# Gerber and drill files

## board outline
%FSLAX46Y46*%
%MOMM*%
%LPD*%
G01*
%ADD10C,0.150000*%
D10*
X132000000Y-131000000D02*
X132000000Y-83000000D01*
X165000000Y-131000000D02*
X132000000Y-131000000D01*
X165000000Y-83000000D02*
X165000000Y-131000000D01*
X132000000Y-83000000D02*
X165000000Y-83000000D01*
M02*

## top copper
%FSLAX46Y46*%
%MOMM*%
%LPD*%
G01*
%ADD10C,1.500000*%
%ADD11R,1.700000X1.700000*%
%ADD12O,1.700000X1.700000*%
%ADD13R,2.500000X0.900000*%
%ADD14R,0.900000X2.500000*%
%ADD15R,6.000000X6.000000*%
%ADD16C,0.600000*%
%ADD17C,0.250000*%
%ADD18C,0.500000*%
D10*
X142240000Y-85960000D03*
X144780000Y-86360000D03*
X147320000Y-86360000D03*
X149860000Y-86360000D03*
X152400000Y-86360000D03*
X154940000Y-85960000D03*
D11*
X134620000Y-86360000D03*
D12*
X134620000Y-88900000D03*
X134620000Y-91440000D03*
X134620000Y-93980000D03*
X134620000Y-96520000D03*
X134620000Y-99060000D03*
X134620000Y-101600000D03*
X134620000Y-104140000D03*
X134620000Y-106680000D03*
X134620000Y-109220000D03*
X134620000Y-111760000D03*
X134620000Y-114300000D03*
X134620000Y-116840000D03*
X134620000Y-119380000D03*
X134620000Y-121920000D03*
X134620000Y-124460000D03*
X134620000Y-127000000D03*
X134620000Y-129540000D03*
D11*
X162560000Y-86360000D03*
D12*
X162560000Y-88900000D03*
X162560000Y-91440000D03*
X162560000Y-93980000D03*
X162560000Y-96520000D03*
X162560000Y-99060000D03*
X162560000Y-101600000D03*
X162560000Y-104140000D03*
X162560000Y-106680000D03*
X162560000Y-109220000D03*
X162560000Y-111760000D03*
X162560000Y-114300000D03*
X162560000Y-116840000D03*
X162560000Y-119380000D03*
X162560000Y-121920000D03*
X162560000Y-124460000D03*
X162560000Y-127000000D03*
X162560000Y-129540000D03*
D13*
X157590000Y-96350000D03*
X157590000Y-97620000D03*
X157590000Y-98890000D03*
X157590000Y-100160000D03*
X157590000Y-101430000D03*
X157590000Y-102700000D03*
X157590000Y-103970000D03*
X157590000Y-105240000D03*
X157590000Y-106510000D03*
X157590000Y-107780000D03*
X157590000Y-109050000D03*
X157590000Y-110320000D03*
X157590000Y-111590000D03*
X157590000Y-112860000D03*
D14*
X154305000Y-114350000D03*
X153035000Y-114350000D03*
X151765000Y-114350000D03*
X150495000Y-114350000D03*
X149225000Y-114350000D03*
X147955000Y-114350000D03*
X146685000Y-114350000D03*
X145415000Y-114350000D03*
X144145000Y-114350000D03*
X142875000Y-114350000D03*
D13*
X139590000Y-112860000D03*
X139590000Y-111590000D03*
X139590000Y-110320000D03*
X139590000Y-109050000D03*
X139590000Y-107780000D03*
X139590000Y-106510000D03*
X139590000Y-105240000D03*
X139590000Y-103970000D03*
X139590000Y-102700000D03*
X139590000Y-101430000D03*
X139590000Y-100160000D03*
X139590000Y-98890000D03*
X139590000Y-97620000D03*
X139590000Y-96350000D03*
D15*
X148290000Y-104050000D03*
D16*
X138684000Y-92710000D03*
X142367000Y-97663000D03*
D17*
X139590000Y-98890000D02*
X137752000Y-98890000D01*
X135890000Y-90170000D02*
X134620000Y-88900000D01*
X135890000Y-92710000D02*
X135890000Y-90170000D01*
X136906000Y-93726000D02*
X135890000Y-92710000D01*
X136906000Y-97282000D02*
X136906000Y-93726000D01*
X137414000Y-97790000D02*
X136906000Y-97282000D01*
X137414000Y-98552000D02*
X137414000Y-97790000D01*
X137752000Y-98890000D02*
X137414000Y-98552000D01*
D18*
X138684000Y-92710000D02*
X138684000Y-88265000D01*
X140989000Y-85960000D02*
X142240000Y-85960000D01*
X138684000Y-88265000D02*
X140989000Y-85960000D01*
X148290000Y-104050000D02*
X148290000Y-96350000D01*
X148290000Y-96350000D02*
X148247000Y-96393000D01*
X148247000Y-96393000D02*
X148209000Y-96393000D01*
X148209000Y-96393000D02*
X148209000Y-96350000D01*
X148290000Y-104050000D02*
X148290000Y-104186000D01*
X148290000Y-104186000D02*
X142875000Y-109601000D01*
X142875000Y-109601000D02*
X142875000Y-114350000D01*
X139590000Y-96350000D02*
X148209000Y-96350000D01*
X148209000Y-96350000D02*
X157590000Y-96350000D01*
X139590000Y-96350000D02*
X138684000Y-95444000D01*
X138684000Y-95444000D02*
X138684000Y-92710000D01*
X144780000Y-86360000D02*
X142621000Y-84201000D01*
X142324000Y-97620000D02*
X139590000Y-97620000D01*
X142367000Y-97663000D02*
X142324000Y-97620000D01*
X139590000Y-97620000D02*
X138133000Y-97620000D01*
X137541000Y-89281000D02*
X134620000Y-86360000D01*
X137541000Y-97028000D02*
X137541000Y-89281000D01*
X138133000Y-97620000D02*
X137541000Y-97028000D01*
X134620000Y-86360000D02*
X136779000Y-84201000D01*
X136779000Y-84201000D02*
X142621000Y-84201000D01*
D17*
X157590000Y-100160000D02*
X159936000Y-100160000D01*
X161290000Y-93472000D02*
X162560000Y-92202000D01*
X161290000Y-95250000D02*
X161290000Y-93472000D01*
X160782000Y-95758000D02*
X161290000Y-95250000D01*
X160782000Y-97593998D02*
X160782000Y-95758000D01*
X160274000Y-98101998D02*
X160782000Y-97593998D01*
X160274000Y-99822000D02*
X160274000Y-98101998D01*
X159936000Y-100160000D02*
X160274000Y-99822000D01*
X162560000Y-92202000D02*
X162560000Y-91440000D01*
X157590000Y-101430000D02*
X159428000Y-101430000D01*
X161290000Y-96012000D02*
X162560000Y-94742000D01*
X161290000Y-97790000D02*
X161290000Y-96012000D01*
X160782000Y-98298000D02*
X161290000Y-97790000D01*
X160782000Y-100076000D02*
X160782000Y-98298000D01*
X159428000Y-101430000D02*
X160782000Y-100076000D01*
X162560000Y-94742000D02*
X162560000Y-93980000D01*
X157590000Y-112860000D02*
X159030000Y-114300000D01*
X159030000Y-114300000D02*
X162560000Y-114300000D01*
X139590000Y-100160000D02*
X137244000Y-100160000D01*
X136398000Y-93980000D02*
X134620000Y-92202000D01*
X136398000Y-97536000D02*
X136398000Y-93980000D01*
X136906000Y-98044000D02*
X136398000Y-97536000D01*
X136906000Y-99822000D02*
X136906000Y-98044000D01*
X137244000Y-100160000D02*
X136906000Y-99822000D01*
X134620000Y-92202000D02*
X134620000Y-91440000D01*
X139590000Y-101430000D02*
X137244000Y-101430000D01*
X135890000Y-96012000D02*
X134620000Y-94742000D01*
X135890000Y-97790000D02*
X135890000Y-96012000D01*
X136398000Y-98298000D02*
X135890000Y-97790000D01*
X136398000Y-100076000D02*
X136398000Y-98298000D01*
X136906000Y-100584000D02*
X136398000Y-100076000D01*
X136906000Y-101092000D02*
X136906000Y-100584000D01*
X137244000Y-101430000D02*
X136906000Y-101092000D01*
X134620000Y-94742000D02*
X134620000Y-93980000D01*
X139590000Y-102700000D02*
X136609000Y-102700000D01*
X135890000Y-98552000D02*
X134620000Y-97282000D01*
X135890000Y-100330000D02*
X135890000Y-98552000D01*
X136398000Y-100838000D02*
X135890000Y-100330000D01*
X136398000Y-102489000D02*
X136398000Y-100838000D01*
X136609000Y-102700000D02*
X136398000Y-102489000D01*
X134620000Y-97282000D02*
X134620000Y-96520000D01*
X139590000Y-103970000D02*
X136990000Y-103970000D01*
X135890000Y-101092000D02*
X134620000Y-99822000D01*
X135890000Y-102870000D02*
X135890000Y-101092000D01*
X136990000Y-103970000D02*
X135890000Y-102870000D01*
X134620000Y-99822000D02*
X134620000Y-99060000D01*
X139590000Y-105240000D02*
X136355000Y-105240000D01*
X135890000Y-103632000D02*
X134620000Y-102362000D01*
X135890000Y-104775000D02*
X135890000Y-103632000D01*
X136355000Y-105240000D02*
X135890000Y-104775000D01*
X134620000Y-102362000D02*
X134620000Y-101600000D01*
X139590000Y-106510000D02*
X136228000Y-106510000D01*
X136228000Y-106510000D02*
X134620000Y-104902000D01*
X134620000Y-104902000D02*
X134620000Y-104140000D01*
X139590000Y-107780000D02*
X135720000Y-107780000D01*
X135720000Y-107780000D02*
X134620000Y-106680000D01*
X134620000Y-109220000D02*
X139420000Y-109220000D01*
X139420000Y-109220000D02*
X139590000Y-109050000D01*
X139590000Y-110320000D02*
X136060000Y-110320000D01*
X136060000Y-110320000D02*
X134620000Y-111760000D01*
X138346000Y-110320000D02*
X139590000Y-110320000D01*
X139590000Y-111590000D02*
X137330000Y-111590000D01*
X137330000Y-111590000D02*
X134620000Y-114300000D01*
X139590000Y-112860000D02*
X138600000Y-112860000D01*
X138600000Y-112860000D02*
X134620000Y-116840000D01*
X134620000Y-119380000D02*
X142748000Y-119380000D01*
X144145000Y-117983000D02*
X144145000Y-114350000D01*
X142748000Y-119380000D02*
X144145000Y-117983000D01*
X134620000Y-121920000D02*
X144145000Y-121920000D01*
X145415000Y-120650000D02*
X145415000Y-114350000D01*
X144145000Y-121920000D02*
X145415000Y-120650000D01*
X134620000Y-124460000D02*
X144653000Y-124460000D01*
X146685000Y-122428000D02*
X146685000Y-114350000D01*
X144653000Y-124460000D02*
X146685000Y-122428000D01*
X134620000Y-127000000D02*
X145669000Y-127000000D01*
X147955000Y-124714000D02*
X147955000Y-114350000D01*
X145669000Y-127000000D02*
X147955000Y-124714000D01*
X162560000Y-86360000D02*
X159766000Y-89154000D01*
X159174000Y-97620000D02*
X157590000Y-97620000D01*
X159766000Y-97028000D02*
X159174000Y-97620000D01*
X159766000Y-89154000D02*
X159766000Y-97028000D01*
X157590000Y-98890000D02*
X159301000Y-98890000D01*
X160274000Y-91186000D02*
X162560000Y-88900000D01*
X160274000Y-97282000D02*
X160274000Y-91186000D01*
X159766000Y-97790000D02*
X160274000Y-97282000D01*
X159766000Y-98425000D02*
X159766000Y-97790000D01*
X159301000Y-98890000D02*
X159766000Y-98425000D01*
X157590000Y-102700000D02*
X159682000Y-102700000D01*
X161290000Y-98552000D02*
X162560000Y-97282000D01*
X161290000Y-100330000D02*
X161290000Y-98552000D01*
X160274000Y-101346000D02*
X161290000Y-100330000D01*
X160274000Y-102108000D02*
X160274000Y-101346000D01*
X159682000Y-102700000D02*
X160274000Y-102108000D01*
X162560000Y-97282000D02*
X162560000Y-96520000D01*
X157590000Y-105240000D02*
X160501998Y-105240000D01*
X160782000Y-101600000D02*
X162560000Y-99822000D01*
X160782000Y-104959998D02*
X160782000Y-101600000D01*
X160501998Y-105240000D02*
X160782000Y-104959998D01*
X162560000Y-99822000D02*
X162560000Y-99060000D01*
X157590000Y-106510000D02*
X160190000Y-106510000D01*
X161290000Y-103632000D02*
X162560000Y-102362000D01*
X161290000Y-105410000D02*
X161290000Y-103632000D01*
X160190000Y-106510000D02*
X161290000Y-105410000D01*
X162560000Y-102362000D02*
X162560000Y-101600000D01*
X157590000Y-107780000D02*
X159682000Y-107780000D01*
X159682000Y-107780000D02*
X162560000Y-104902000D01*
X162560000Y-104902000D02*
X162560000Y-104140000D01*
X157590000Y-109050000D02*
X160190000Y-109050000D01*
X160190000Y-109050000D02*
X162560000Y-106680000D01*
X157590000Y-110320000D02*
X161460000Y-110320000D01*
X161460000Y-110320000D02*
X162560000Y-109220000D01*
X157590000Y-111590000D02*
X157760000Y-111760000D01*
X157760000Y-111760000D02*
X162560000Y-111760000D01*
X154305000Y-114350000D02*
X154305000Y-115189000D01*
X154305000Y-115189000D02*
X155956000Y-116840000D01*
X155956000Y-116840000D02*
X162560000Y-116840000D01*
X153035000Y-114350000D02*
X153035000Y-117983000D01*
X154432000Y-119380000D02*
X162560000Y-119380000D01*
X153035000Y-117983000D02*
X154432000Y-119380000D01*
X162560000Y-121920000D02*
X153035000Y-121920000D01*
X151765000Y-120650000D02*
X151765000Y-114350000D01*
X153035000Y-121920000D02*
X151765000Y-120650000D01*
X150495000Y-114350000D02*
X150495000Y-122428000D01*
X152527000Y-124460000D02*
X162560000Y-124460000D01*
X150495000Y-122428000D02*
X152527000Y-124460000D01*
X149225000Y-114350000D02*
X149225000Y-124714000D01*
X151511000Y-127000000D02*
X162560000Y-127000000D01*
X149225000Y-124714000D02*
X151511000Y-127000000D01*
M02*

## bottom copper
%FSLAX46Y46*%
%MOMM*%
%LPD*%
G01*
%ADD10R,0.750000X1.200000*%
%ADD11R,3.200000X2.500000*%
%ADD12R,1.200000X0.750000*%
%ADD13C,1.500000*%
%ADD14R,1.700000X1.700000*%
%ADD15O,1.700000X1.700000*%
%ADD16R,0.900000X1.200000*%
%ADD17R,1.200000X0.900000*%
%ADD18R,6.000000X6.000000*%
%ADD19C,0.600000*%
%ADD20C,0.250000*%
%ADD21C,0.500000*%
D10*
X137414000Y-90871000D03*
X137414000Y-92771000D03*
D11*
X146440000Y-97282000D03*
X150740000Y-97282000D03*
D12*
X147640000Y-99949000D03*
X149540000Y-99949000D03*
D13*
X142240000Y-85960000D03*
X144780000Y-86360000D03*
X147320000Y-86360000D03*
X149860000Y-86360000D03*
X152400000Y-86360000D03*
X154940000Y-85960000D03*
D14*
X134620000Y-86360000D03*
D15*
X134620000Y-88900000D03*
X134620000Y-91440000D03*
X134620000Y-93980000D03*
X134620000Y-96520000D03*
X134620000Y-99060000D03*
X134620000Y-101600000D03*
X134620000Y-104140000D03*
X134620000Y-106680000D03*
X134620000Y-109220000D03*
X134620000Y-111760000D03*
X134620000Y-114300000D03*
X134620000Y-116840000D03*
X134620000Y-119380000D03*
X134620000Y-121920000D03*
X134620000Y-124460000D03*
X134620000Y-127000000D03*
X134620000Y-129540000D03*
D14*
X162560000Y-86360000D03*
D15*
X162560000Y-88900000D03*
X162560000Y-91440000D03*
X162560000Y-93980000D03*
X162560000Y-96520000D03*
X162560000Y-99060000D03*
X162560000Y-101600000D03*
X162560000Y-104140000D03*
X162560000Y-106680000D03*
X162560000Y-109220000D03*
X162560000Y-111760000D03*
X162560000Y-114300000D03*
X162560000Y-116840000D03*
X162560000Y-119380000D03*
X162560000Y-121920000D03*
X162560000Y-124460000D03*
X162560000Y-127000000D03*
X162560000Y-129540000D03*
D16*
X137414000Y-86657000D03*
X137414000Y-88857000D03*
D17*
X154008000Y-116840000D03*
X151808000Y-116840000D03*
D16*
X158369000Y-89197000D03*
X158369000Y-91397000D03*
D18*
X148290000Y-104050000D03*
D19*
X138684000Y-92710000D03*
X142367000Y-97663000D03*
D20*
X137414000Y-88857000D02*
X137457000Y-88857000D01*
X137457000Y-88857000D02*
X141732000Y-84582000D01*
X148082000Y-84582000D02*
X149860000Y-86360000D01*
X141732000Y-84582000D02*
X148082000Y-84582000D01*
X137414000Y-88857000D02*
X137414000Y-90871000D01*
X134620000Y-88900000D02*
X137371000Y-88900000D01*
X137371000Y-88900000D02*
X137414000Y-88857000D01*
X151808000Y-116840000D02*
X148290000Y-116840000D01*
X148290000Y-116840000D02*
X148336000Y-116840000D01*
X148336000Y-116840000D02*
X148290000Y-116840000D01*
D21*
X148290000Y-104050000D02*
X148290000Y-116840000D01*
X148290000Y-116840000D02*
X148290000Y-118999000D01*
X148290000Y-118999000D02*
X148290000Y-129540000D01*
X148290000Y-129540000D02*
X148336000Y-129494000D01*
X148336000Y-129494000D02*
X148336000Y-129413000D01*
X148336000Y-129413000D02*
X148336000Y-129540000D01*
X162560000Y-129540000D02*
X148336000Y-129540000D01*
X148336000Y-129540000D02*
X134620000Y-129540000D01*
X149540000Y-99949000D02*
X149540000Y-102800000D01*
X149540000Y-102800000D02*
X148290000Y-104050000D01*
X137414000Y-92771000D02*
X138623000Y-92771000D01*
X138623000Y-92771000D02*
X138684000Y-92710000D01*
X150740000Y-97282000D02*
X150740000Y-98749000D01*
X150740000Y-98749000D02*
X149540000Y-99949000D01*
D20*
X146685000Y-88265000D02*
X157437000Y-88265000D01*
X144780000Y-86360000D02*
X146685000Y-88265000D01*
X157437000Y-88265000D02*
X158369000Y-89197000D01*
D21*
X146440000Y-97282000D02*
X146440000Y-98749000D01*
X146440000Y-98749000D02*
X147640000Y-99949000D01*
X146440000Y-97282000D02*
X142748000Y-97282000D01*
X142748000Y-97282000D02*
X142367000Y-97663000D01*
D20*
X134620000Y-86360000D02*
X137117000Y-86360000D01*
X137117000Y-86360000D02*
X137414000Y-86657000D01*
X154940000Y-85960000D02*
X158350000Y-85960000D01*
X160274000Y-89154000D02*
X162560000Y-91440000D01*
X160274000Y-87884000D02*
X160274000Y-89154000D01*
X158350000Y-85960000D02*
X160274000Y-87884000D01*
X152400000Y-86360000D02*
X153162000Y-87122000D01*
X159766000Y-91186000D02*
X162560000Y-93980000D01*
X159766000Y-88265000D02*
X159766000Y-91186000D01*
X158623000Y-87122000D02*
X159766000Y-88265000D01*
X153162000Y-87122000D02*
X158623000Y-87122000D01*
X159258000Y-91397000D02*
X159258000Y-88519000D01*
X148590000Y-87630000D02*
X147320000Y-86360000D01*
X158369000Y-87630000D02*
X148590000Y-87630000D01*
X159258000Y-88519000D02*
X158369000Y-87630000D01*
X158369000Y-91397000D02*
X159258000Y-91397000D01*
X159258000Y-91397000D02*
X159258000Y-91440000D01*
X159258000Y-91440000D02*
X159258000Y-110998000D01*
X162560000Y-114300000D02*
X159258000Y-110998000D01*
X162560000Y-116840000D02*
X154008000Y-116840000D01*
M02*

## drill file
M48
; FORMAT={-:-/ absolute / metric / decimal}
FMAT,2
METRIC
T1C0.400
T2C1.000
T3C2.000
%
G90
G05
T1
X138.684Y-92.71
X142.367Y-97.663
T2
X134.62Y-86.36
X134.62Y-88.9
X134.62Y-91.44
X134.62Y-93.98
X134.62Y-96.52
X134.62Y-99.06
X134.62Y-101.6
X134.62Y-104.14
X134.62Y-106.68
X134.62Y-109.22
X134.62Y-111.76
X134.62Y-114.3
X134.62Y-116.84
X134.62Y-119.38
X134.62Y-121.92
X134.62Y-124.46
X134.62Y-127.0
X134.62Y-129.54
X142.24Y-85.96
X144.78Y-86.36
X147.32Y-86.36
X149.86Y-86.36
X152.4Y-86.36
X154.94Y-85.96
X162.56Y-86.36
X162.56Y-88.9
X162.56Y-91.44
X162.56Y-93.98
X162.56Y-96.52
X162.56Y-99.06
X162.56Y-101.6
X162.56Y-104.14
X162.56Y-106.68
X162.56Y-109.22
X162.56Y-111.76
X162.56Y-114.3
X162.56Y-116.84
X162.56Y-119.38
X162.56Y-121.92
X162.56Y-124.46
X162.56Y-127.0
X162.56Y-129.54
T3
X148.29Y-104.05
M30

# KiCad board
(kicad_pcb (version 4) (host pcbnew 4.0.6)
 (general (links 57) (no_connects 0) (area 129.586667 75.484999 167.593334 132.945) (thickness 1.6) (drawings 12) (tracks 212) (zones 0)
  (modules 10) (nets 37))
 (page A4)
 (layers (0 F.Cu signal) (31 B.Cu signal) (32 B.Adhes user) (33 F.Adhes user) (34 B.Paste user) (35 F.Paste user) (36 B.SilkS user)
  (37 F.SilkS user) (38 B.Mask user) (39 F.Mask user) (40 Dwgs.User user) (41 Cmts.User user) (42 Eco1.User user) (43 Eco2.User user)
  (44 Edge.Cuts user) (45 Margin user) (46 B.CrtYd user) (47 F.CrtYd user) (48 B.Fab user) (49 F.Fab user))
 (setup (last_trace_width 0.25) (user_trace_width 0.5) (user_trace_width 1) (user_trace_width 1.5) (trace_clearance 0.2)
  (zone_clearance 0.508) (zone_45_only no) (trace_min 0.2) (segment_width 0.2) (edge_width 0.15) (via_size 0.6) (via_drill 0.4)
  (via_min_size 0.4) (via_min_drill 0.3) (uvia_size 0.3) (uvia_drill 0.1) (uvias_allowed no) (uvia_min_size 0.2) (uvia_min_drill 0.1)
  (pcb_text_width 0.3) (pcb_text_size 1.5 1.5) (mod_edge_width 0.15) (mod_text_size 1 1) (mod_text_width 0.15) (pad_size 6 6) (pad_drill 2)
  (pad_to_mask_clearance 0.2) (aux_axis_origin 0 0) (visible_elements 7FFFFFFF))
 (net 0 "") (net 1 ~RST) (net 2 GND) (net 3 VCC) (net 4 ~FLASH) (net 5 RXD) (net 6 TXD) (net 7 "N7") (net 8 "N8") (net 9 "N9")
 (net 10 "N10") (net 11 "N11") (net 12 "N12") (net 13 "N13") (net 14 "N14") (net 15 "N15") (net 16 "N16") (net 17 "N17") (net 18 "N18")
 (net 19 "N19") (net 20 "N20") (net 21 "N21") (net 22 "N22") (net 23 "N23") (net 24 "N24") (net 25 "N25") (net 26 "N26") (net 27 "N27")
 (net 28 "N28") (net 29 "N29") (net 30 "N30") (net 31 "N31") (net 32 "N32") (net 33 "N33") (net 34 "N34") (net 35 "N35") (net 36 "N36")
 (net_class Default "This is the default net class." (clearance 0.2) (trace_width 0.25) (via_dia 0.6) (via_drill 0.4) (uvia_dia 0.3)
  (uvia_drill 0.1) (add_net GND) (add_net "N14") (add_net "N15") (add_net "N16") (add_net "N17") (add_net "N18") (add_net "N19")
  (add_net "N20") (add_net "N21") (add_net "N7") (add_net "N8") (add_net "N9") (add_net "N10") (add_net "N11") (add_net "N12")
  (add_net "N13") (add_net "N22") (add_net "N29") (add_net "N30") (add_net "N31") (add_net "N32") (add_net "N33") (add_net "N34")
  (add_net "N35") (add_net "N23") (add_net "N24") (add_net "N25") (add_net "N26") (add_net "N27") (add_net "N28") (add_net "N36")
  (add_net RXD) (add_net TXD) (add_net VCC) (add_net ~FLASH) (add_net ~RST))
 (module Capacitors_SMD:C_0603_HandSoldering (layer B.Cu) (at 137.414 91.821 270)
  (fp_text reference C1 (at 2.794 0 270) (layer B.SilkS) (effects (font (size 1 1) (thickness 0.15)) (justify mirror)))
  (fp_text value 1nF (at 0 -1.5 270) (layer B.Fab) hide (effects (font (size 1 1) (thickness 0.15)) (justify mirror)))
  (pad 1 smd rect (at -0.95 0 270) (size 1.2 0.75) (layers B.Cu B.Paste B.Mask) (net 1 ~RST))
  (pad 2 smd rect (at 0.95 0 270) (size 1.2 0.75) (layers B.Cu B.Paste B.Mask) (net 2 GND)))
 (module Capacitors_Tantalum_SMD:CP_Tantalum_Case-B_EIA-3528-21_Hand (layer B.Cu) (at 148.59 97.282)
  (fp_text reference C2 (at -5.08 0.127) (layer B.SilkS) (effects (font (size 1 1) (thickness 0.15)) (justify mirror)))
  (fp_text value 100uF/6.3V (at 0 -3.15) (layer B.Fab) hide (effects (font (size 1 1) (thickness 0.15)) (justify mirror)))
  (pad 1 smd rect (at -2.15 0) (size 3.2 2.5) (layers B.Cu B.Paste B.Mask) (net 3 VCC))
  (pad 2 smd rect (at 2.15 0) (size 3.2 2.5) (layers B.Cu B.Paste B.Mask) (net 2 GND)))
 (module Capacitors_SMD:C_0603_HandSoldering (layer B.Cu) (at 148.59 99.949)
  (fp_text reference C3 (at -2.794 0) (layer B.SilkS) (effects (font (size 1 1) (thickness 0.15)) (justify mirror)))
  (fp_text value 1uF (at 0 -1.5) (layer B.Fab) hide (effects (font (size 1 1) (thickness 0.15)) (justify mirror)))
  (pad 1 smd rect (at -0.95 0) (size 1.2 0.75) (layers B.Cu B.Paste B.Mask) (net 3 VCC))
  (pad 2 smd rect (at 0.95 0) (size 1.2 0.75) (layers B.Cu B.Paste B.Mask) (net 2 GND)))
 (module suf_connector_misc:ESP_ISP (layer F.Cu) (at 142.24 86.36 90)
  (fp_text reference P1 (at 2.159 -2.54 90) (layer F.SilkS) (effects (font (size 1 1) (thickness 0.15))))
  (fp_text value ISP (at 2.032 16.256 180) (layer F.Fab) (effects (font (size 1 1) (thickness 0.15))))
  (pad 1 thru_hole circle (at 0.4 0 90) (size 1.5 1.5) (drill 1) (layers *.Cu *.Mask) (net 2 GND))
  (pad 2 thru_hole circle (at 0 2.54 90) (size 1.5 1.5) (drill 1) (layers *.Cu *.Mask) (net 3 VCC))
  (pad 3 thru_hole circle (at 0 5.08 90) (size 1.5 1.5) (drill 1) (layers *.Cu *.Mask) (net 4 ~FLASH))
  (pad 4 thru_hole circle (at 0 7.62 90) (size 1.5 1.5) (drill 1) (layers *.Cu *.Mask) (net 1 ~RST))
  (pad 5 thru_hole circle (at 0 10.16 90) (size 1.5 1.5) (drill 1) (layers *.Cu *.Mask) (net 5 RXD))
  (pad 6 thru_hole circle (at 0.4 12.7 90) (size 1.5 1.5) (drill 1) (layers *.Cu *.Mask) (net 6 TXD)))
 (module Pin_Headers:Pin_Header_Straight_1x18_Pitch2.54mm (layer F.Cu) (at 134.62 86.36)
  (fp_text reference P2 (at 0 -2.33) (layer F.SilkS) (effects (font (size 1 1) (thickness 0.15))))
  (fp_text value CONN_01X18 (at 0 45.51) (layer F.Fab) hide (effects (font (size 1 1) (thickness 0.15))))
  (pad 1 thru_hole rect (at 0 0) (size 1.7 1.7) (drill 1) (layers *.Cu *.Mask) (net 3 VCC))
  (pad 2 thru_hole oval (at 0 2.54) (size 1.7 1.7) (drill 1) (layers *.Cu *.Mask) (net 1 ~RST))
  (pad 3 thru_hole oval (at 0 5.08) (size 1.7 1.7) (drill 1) (layers *.Cu *.Mask) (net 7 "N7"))
  (pad 4 thru_hole oval (at 0 7.62) (size 1.7 1.7) (drill 1) (layers *.Cu *.Mask) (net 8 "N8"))
  (pad 5 thru_hole oval (at 0 10.16) (size 1.7 1.7) (drill 1) (layers *.Cu *.Mask) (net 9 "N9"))
  (pad 6 thru_hole oval (at 0 12.7) (size 1.7 1.7) (drill 1) (layers *.Cu *.Mask) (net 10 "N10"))
  (pad 7 thru_hole oval (at 0 15.24) (size 1.7 1.7) (drill 1) (layers *.Cu *.Mask) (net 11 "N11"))
  (pad 8 thru_hole oval (at 0 17.78) (size 1.7 1.7) (drill 1) (layers *.Cu *.Mask) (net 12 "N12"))
  (pad 9 thru_hole oval (at 0 20.32) (size 1.7 1.7) (drill 1) (layers *.Cu *.Mask) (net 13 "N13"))
  (pad 10 thru_hole oval (at 0 22.86) (size 1.7 1.7) (drill 1) (layers *.Cu *.Mask) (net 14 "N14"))
  (pad 11 thru_hole oval (at 0 25.4) (size 1.7 1.7) (drill 1) (layers *.Cu *.Mask) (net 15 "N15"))
  (pad 12 thru_hole oval (at 0 27.94) (size 1.7 1.7) (drill 1) (layers *.Cu *.Mask) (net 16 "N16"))
  (pad 13 thru_hole oval (at 0 30.48) (size 1.7 1.7) (drill 1) (layers *.Cu *.Mask) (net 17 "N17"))
  (pad 14 thru_hole oval (at 0 33.02) (size 1.7 1.7) (drill 1) (layers *.Cu *.Mask) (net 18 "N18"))
  (pad 15 thru_hole oval (at 0 35.56) (size 1.7 1.7) (drill 1) (layers *.Cu *.Mask) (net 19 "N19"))
  (pad 16 thru_hole oval (at 0 38.1) (size 1.7 1.7) (drill 1) (layers *.Cu *.Mask) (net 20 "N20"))
  (pad 17 thru_hole oval (at 0 40.64) (size 1.7 1.7) (drill 1) (layers *.Cu *.Mask) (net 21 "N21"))
  (pad 18 thru_hole oval (at 0 43.18) (size 1.7 1.7) (drill 1) (layers *.Cu *.Mask) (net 2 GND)))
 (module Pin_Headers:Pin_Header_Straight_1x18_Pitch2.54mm (layer F.Cu) (at 162.56 86.36)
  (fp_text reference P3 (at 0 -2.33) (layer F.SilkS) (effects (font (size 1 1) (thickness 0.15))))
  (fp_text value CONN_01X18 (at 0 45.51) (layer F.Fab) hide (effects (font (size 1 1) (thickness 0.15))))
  (pad 1 thru_hole rect (at 0 0) (size 1.7 1.7) (drill 1) (layers *.Cu *.Mask) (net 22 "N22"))
  (pad 2 thru_hole oval (at 0 2.54) (size 1.7 1.7) (drill 1) (layers *.Cu *.Mask) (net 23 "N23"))
  (pad 3 thru_hole oval (at 0 5.08) (size 1.7 1.7) (drill 1) (layers *.Cu *.Mask) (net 6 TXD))
  (pad 4 thru_hole oval (at 0 7.62) (size 1.7 1.7) (drill 1) (layers *.Cu *.Mask) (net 5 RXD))
  (pad 5 thru_hole oval (at 0 10.16) (size 1.7 1.7) (drill 1) (layers *.Cu *.Mask) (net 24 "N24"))
  (pad 6 thru_hole oval (at 0 12.7) (size 1.7 1.7) (drill 1) (layers *.Cu *.Mask) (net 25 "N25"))
  (pad 7 thru_hole oval (at 0 15.24) (size 1.7 1.7) (drill 1) (layers *.Cu *.Mask) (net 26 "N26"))
  (pad 8 thru_hole oval (at 0 17.78) (size 1.7 1.7) (drill 1) (layers *.Cu *.Mask) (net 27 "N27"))
  (pad 9 thru_hole oval (at 0 20.32) (size 1.7 1.7) (drill 1) (layers *.Cu *.Mask) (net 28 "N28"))
  (pad 10 thru_hole oval (at 0 22.86) (size 1.7 1.7) (drill 1) (layers *.Cu *.Mask) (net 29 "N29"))
  (pad 11 thru_hole oval (at 0 25.4) (size 1.7 1.7) (drill 1) (layers *.Cu *.Mask) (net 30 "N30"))
  (pad 12 thru_hole oval (at 0 27.94) (size 1.7 1.7) (drill 1) (layers *.Cu *.Mask) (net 4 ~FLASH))
  (pad 13 thru_hole oval (at 0 30.48) (size 1.7 1.7) (drill 1) (layers *.Cu *.Mask) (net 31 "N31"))
  (pad 14 thru_hole oval (at 0 33.02) (size 1.7 1.7) (drill 1) (layers *.Cu *.Mask) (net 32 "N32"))
  (pad 15 thru_hole oval (at 0 35.56) (size 1.7 1.7) (drill 1) (layers *.Cu *.Mask) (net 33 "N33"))
  (pad 16 thru_hole oval (at 0 38.1) (size 1.7 1.7) (drill 1) (layers *.Cu *.Mask) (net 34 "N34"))
  (pad 17 thru_hole oval (at 0 40.64) (size 1.7 1.7) (drill 1) (layers *.Cu *.Mask) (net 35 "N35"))
  (pad 18 thru_hole oval (at 0 43.18) (size 1.7 1.7) (drill 1) (layers *.Cu *.Mask) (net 2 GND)))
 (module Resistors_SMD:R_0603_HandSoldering (layer B.Cu) (at 137.414 87.757 270)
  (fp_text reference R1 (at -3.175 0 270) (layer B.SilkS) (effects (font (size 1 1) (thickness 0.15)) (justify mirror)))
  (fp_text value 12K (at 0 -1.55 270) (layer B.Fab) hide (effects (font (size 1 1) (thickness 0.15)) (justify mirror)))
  (pad 1 smd rect (at -1.1 0 270) (size 1.2 0.9) (layers B.Cu B.Paste B.Mask) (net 3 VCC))
  (pad 2 smd rect (at 1.1 0 270) (size 1.2 0.9) (layers B.Cu B.Paste B.Mask) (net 1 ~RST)))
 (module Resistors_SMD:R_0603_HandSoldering (layer B.Cu) (at 152.908 116.84 180)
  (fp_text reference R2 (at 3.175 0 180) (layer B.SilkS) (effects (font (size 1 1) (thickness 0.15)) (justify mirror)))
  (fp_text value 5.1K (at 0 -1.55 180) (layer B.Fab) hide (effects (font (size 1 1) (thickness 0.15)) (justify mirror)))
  (pad 1 smd rect (at -1.1 0 180) (size 1.2 0.9) (layers B.Cu B.Paste B.Mask) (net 31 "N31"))
  (pad 2 smd rect (at 1.1 0 180) (size 1.2 0.9) (layers B.Cu B.Paste B.Mask) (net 2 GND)))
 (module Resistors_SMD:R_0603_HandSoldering (layer B.Cu) (at 158.369 90.297 270)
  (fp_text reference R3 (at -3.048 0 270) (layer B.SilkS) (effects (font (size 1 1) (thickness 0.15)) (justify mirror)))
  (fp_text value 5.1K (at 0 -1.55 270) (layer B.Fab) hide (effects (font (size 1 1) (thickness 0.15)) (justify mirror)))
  (pad 1 smd rect (at -1.1 0 270) (size 1.2 0.9) (layers B.Cu B.Paste B.Mask) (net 3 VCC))
  (pad 2 smd rect (at 1.1 0 270) (size 1.2 0.9) (layers B.Cu B.Paste B.Mask) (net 4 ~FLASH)))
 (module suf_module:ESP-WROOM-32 (layer F.Cu) (at 148.59 101.6 180)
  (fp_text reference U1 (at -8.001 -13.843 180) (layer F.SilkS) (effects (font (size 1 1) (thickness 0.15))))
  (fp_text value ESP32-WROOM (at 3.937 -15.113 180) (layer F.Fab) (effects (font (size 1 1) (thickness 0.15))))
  (pad 38 smd rect (at -9 5.25 180) (size 2.5 0.9) (layers F.Cu F.Paste F.Mask) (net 2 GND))
  (pad 37 smd rect (at -9 3.98 180) (size 2.5 0.9) (layers F.Cu F.Paste F.Mask) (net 22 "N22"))
  (pad 36 smd rect (at -9 2.71 180) (size 2.5 0.9) (layers F.Cu F.Paste F.Mask) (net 23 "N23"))
  (pad 35 smd rect (at -9 1.44 180) (size 2.5 0.9) (layers F.Cu F.Paste F.Mask) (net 6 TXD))
  (pad 34 smd rect (at -9 0.17 180) (size 2.5 0.9) (layers F.Cu F.Paste F.Mask) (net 5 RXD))
  (pad 33 smd rect (at -9 -1.1 180) (size 2.5 0.9) (layers F.Cu F.Paste F.Mask) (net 24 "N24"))
  (pad 32 smd rect (at -9 -2.37 180) (size 2.5 0.9) (layers F.Cu F.Paste F.Mask) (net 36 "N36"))
  (pad 31 smd rect (at -9 -3.64 180) (size 2.5 0.9) (layers F.Cu F.Paste F.Mask) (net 25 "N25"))
  (pad 30 smd rect (at -9 -4.91 180) (size 2.5 0.9) (layers F.Cu F.Paste F.Mask) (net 26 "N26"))
  (pad 29 smd rect (at -9 -6.18 180) (size 2.5 0.9) (layers F.Cu F.Paste F.Mask) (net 27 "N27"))
  (pad 28 smd rect (at -9 -7.45 180) (size 2.5 0.9) (layers F.Cu F.Paste F.Mask) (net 28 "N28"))
  (pad 27 smd rect (at -9 -8.72 180) (size 2.5 0.9) (layers F.Cu F.Paste F.Mask) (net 29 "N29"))
  (pad 26 smd rect (at -9 -9.99 180) (size 2.5 0.9) (layers F.Cu F.Paste F.Mask) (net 30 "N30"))
  (pad 25 smd rect (at -9 -11.26 180) (size 2.5 0.9) (layers F.Cu F.Paste F.Mask) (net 4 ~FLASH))
  (pad 24 smd rect (at -5.715 -12.75 180) (size 0.9 2.5) (layers F.Cu F.Paste F.Mask) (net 31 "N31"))
  (pad 23 smd rect (at -4.445 -12.75 180) (size 0.9 2.5) (layers F.Cu F.Paste F.Mask) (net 32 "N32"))
  (pad 22 smd rect (at -3.175 -12.75 180) (size 0.9 2.5) (layers F.Cu F.Paste F.Mask) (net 33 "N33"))
  (pad 21 smd rect (at -1.905 -12.75 180) (size 0.9 2.5) (layers F.Cu F.Paste F.Mask) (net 34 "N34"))
  (pad 20 smd rect (at -0.635 -12.75 180) (size 0.9 2.5) (layers F.Cu F.Paste F.Mask) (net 35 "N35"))
  (pad 19 smd rect (at 0.635 -12.75 180) (size 0.9 2.5) (layers F.Cu F.Paste F.Mask) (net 21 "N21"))
  (pad 18 smd rect (at 1.905 -12.75 180) (size 0.9 2.5) (layers F.Cu F.Paste F.Mask) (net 20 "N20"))
  (pad 17 smd rect (at 3.175 -12.75 180) (size 0.9 2.5) (layers F.Cu F.Paste F.Mask) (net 19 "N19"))
  (pad 16 smd rect (at 4.445 -12.75 180) (size 0.9 2.5) (layers F.Cu F.Paste F.Mask) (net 18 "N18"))
  (pad 15 smd rect (at 5.715 -12.75 180) (size 0.9 2.5) (layers F.Cu F.Paste F.Mask) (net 2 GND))
  (pad 14 smd rect (at 9 -11.26 180) (size 2.5 0.9) (layers F.Cu F.Paste F.Mask) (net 17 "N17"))
  (pad 13 smd rect (at 9 -9.99 180) (size 2.5 0.9) (layers F.Cu F.Paste F.Mask) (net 16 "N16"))
  (pad 12 smd rect (at 9 -8.72 180) (size 2.5 0.9) (layers F.Cu F.Paste F.Mask) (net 15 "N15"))
  (pad 11 smd rect (at 9 -7.45 180) (size 2.5 0.9) (layers F.Cu F.Paste F.Mask) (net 14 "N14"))
  (pad 10 smd rect (at 9 -6.18 180) (size 2.5 0.9) (layers F.Cu F.Paste F.Mask) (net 13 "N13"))
  (pad 9 smd rect (at 9 -4.91 180) (size 2.5 0.9) (layers F.Cu F.Paste F.Mask) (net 12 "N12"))
  (pad 8 smd rect (at 9 -3.64 180) (size 2.5 0.9) (layers F.Cu F.Paste F.Mask) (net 11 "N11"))
  (pad 7 smd rect (at 9 -2.37 180) (size 2.5 0.9) (layers F.Cu F.Paste F.Mask) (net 10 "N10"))
  (pad 6 smd rect (at 9 -1.1 180) (size 2.5 0.9) (layers F.Cu F.Paste F.Mask) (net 9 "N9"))
  (pad 5 smd rect (at 9 0.17 180) (size 2.5 0.9) (layers F.Cu F.Paste F.Mask) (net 8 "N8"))
  (pad 4 smd rect (at 9 1.44 180) (size 2.5 0.9) (layers F.Cu F.Paste F.Mask) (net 7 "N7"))
  (pad 3 smd rect (at 9 2.71 180) (size 2.5 0.9) (layers F.Cu F.Paste F.Mask) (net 1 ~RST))
  (pad 2 smd rect (at 9 3.98 180) (size 2.5 0.9) (layers F.Cu F.Paste F.Mask) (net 3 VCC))
  (pad 1 smd rect (at 9 5.25 180) (size 2.5 0.9) (layers F.Cu F.Paste F.Mask) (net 2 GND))
  (pad 39 thru_hole rect (at 0.3 -2.45 180) (size 6 6) (drill 2) (layers *.Cu *.Mask F.SilkS) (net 2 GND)))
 (gr_line (start 132 131) (end 132 83) (angle 90) (layer Edge.Cuts) (width 0.15))
 (gr_line (start 165 131) (end 132 131) (angle 90) (layer Edge.Cuts) (width 0.15))
 (gr_line (start 165 83) (end 165 131) (angle 90) (layer Edge.Cuts) (width 0.15))
 (gr_line (start 132 83) (end 165 83) (angle 90) (layer Edge.Cuts) (width 0.15))
 (segment (start 137.414 88.857) (end 137.457 88.857) (width 0.25) (layer B.Cu) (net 1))
 (segment (start 137.457 88.857) (end 141.732 84.582) (width 0.25) (layer B.Cu) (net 1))
 (segment (start 148.082 84.582) (end 149.86 86.36) (width 0.25) (layer B.Cu) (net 1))
 (segment (start 141.732 84.582) (end 148.082 84.582) (width 0.25) (layer B.Cu) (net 1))
 (segment (start 139.59 98.89) (end 137.752 98.89) (width 0.25) (layer F.Cu) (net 1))
 (segment (start 135.89 90.17) (end 134.62 88.9) (width 0.25) (layer F.Cu) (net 1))
 (segment (start 135.89 92.71) (end 135.89 90.17) (width 0.25) (layer F.Cu) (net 1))
 (segment (start 136.906 93.726) (end 135.89 92.71) (width 0.25) (layer F.Cu) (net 1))
 (segment (start 136.906 97.282) (end 136.906 93.726) (width 0.25) (layer F.Cu) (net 1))
 (segment (start 137.414 97.79) (end 136.906 97.282) (width 0.25) (layer F.Cu) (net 1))
 (segment (start 137.414 98.552) (end 137.414 97.79) (width 0.25) (layer F.Cu) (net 1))
 (segment (start 137.752 98.89) (end 137.414 98.552) (width 0.25) (layer F.Cu) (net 1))
 (segment (start 137.414 88.857) (end 137.414 90.871) (width 0.25) (layer B.Cu) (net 1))
 (segment (start 134.62 88.9) (end 137.371 88.9) (width 0.25) (layer B.Cu) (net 1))
 (segment (start 137.371 88.9) (end 137.414 88.857) (width 0.25) (layer B.Cu) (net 1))
 (segment (start 151.808 116.84) (end 148.29 116.84) (width 0.25) (layer B.Cu) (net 2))
 (segment (start 148.29 116.84) (end 148.336 116.84) (width 0.25) (layer B.Cu) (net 2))
 (segment (start 148.336 116.84) (end 148.29 116.84) (width 0.25) (layer B.Cu) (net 2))
 (segment (start 138.684 92.71) (end 138.684 88.265) (width 0.5) (layer F.Cu) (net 2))
 (segment (start 140.989 85.96) (end 142.24 85.96) (width 0.5) (layer F.Cu) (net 2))
 (segment (start 138.684 88.265) (end 140.989 85.96) (width 0.5) (layer F.Cu) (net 2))
 (segment (start 148.29 104.05) (end 148.29 96.35) (width 0.5) (layer F.Cu) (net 2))
 (segment (start 148.29 96.35) (end 148.247 96.393) (width 0.5) (layer F.Cu) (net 2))
 (segment (start 148.247 96.393) (end 148.209 96.393) (width 0.5) (layer F.Cu) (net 2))
 (segment (start 148.209 96.393) (end 148.209 96.35) (width 0.5) (layer F.Cu) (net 2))
 (segment (start 148.29 104.05) (end 148.29 116.84) (width 0.5) (layer B.Cu) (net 2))
 (segment (start 148.29 116.84) (end 148.29 118.999) (width 0.5) (layer B.Cu) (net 2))
 (segment (start 148.29 118.999) (end 148.29 129.54) (width 0.5) (layer B.Cu) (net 2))
 (segment (start 148.29 129.54) (end 148.336 129.494) (width 0.5) (layer B.Cu) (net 2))
 (segment (start 148.336 129.494) (end 148.336 129.413) (width 0.5) (layer B.Cu) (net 2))
 (segment (start 148.336 129.413) (end 148.336 129.54) (width 0.5) (layer B.Cu) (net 2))
 (segment (start 162.56 129.54) (end 148.336 129.54) (width 0.5) (layer B.Cu) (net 2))
 (segment (start 148.336 129.54) (end 134.62 129.54) (width 0.5) (layer B.Cu) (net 2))
 (segment (start 148.29 104.05) (end 148.29 104.186) (width 0.5) (layer F.Cu) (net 2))
 (segment (start 148.29 104.186) (end 142.875 109.601) (width 0.5) (layer F.Cu) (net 2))
 (segment (start 142.875 109.601) (end 142.875 114.35) (width 0.5) (layer F.Cu) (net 2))
 (segment (start 149.54 99.949) (end 149.54 102.8) (width 0.5) (layer B.Cu) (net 2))
 (segment (start 149.54 102.8) (end 148.29 104.05) (width 0.5) (layer B.Cu) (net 2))
 (segment (start 137.414 92.771) (end 138.623 92.771) (width 0.5) (layer B.Cu) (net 2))
 (via (at 138.684 92.71) (size 0.6) (drill 0.4) (layers F.Cu B.Cu) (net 2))
 (segment (start 138.623 92.771) (end 138.684 92.71) (width 0.5) (layer B.Cu) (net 2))
 (segment (start 139.59 96.35) (end 148.209 96.35) (width 0.5) (layer F.Cu) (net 2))
 (segment (start 148.209 96.35) (end 157.59 96.35) (width 0.5) (layer F.Cu) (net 2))
 (segment (start 150.74 97.282) (end 150.74 98.749) (width 0.5) (layer B.Cu) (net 2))
 (segment (start 150.74 98.749) (end 149.54 99.949) (width 0.5) (layer B.Cu) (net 2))
 (segment (start 139.59 96.35) (end 138.684 95.444) (width 0.5) (layer F.Cu) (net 2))
 (segment (start 138.684 95.444) (end 138.684 92.71) (width 0.5) (layer F.Cu) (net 2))
 (segment (start 146.685 88.265) (end 157.437 88.265) (width 0.25) (layer B.Cu) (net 3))
 (segment (start 144.78 86.36) (end 146.685 88.265) (width 0.25) (layer B.Cu) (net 3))
 (segment (start 157.437 88.265) (end 158.369 89.197) (width 0.25) (layer B.Cu) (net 3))
 (segment (start 144.78 86.36) (end 142.621 84.201) (width 0.5) (layer F.Cu) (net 3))
 (segment (start 146.44 97.282) (end 146.44 98.749) (width 0.5) (layer B.Cu) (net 3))
 (segment (start 146.44 98.749) (end 147.64 99.949) (width 0.5) (layer B.Cu) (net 3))
 (segment (start 146.44 97.282) (end 142.748 97.282) (width 0.5) (layer B.Cu) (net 3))
 (segment (start 142.324 97.62) (end 139.59 97.62) (width 0.5) (layer F.Cu) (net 3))
 (segment (start 142.367 97.663) (end 142.324 97.62) (width 0.5) (layer F.Cu) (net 3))
 (via (at 142.367 97.663) (size 0.6) (drill 0.4) (layers F.Cu B.Cu) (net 3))
 (segment (start 142.748 97.282) (end 142.367 97.663) (width 0.5) (layer B.Cu) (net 3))
 (segment (start 139.59 97.62) (end 138.133 97.62) (width 0.5) (layer F.Cu) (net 3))
 (segment (start 137.541 89.281) (end 134.62 86.36) (width 0.5) (layer F.Cu) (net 3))
 (segment (start 137.541 97.028) (end 137.541 89.281) (width 0.5) (layer F.Cu) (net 3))
 (segment (start 138.133 97.62) (end 137.541 97.028) (width 0.5) (layer F.Cu) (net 3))
 (segment (start 134.62 86.36) (end 136.779 84.201) (width 0.5) (layer F.Cu) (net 3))
 (segment (start 136.779 84.201) (end 142.621 84.201) (width 0.5) (layer F.Cu) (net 3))
 (segment (start 134.62 86.36) (end 137.117 86.36) (width 0.25) (layer B.Cu) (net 3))
 (segment (start 137.117 86.36) (end 137.414 86.657) (width 0.25) (layer B.Cu) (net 3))
 (segment (start 154.94 85.96) (end 158.35 85.96) (width 0.25) (layer B.Cu) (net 6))
 (segment (start 160.274 89.154) (end 162.56 91.44) (width 0.25) (layer B.Cu) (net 6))
 (segment (start 160.274 87.884) (end 160.274 89.154) (width 0.25) (layer B.Cu) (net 6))
 (segment (start 158.35 85.96) (end 160.274 87.884) (width 0.25) (layer B.Cu) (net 6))
 (segment (start 157.59 100.16) (end 159.936 100.16) (width 0.25) (layer F.Cu) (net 6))
 (segment (start 161.29 93.472) (end 162.56 92.202) (width 0.25) (layer F.Cu) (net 6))
 (segment (start 161.29 95.25) (end 161.29 93.472) (width 0.25) (layer F.Cu) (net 6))
 (segment (start 160.782 95.758) (end 161.29 95.25) (width 0.25) (layer F.Cu) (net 6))
 (segment (start 160.782 97.593998) (end 160.782 95.758) (width 0.25) (layer F.Cu) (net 6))
 (segment (start 160.274 98.101998) (end 160.782 97.593998) (width 0.25) (layer F.Cu) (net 6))
 (segment (start 160.274 99.822) (end 160.274 98.101998) (width 0.25) (layer F.Cu) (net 6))
 (segment (start 159.936 100.16) (end 160.274 99.822) (width 0.25) (layer F.Cu) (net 6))
 (segment (start 162.56 92.202) (end 162.56 91.44) (width 0.25) (layer F.Cu) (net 6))
 (segment (start 152.4 86.36) (end 153.162 87.122) (width 0.25) (layer B.Cu) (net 5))
 (segment (start 159.766 91.186) (end 162.56 93.98) (width 0.25) (layer B.Cu) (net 5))
 (segment (start 159.766 88.265) (end 159.766 91.186) (width 0.25) (layer B.Cu) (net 5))
 (segment (start 158.623 87.122) (end 159.766 88.265) (width 0.25) (layer B.Cu) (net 5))
 (segment (start 153.162 87.122) (end 158.623 87.122) (width 0.25) (layer B.Cu) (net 5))
 (segment (start 157.59 101.43) (end 159.428 101.43) (width 0.25) (layer F.Cu) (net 5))
 (segment (start 161.29 96.012) (end 162.56 94.742) (width 0.25) (layer F.Cu) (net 5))
 (segment (start 161.29 97.79) (end 161.29 96.012) (width 0.25) (layer F.Cu) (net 5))
 (segment (start 160.782 98.298) (end 161.29 97.79) (width 0.25) (layer F.Cu) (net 5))
 (segment (start 160.782 100.076) (end 160.782 98.298) (width 0.25) (layer F.Cu) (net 5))
 (segment (start 159.428 101.43) (end 160.782 100.076) (width 0.25) (layer F.Cu) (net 5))
 (segment (start 162.56 94.742) (end 162.56 93.98) (width 0.25) (layer F.Cu) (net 5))
 (segment (start 159.258 91.397) (end 159.258 88.519) (width 0.25) (layer B.Cu) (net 4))
 (segment (start 148.59 87.63) (end 147.32 86.36) (width 0.25) (layer B.Cu) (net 4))
 (segment (start 158.369 87.63) (end 148.59 87.63) (width 0.25) (layer B.Cu) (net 4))
 (segment (start 159.258 88.519) (end 158.369 87.63) (width 0.25) (layer B.Cu) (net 4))
 (segment (start 158.369 91.397) (end 159.258 91.397) (width 0.25) (layer B.Cu) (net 4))
 (segment (start 159.258 91.397) (end 159.258 91.44) (width 0.25) (layer B.Cu) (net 4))
 (segment (start 159.258 91.44) (end 159.258 110.998) (width 0.25) (layer B.Cu) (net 4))
 (segment (start 162.56 114.3) (end 159.258 110.998) (width 0.25) (layer B.Cu) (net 4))
 (segment (start 157.59 112.86) (end 159.03 114.3) (width 0.25) (layer F.Cu) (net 4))
 (segment (start 159.03 114.3) (end 162.56 114.3) (width 0.25) (layer F.Cu) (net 4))
 (segment (start 139.59 100.16) (end 137.244 100.16) (width 0.25) (layer F.Cu) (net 7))
 (segment (start 136.398 93.98) (end 134.62 92.202) (width 0.25) (layer F.Cu) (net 7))
 (segment (start 136.398 97.536) (end 136.398 93.98) (width 0.25) (layer F.Cu) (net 7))
 (segment (start 136.906 98.044) (end 136.398 97.536) (width 0.25) (layer F.Cu) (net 7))
 (segment (start 136.906 99.822) (end 136.906 98.044) (width 0.25) (layer F.Cu) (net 7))
 (segment (start 137.244 100.16) (end 136.906 99.822) (width 0.25) (layer F.Cu) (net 7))
 (segment (start 134.62 92.202) (end 134.62 91.44) (width 0.25) (layer F.Cu) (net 7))
 (segment (start 139.59 101.43) (end 137.244 101.43) (width 0.25) (layer F.Cu) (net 8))
 (segment (start 135.89 96.012) (end 134.62 94.742) (width 0.25) (layer F.Cu) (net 8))
 (segment (start 135.89 97.79) (end 135.89 96.012) (width 0.25) (layer F.Cu) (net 8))
 (segment (start 136.398 98.298) (end 135.89 97.79) (width 0.25) (layer F.Cu) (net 8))
 (segment (start 136.398 100.076) (end 136.398 98.298) (width 0.25) (layer F.Cu) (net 8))
 (segment (start 136.906 100.584) (end 136.398 100.076) (width 0.25) (layer F.Cu) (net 8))
 (segment (start 136.906 101.092) (end 136.906 100.584) (width 0.25) (layer F.Cu) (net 8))
 (segment (start 137.244 101.43) (end 136.906 101.092) (width 0.25) (layer F.Cu) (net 8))
 (segment (start 134.62 94.742) (end 134.62 93.98) (width 0.25) (layer F.Cu) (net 8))
 (segment (start 139.59 102.7) (end 136.609 102.7) (width 0.25) (layer F.Cu) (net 9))
 (segment (start 135.89 98.552) (end 134.62 97.282) (width 0.25) (layer F.Cu) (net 9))
 (segment (start 135.89 100.33) (end 135.89 98.552) (width 0.25) (layer F.Cu) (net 9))
 (segment (start 136.398 100.838) (end 135.89 100.33) (width 0.25) (layer F.Cu) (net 9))
 (segment (start 136.398 102.489) (end 136.398 100.838) (width 0.25) (layer F.Cu) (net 9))
 (segment (start 136.609 102.7) (end 136.398 102.489) (width 0.25) (layer F.Cu) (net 9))
 (segment (start 134.62 97.282) (end 134.62 96.52) (width 0.25) (layer F.Cu) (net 9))
 (segment (start 139.59 103.97) (end 136.99 103.97) (width 0.25) (layer F.Cu) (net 10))
 (segment (start 135.89 101.092) (end 134.62 99.822) (width 0.25) (layer F.Cu) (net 10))
 (segment (start 135.89 102.87) (end 135.89 101.092) (width 0.25) (layer F.Cu) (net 10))
 (segment (start 136.99 103.97) (end 135.89 102.87) (width 0.25) (layer F.Cu) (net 10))
 (segment (start 134.62 99.822) (end 134.62 99.06) (width 0.25) (layer F.Cu) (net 10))
 (segment (start 139.59 105.24) (end 136.355 105.24) (width 0.25) (layer F.Cu) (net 11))
 (segment (start 135.89 103.632) (end 134.62 102.362) (width 0.25) (layer F.Cu) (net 11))
 (segment (start 135.89 104.775) (end 135.89 103.632) (width 0.25) (layer F.Cu) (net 11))
 (segment (start 136.355 105.24) (end 135.89 104.775) (width 0.25) (layer F.Cu) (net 11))
 (segment (start 134.62 102.362) (end 134.62 101.6) (width 0.25) (layer F.Cu) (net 11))
 (segment (start 139.59 106.51) (end 136.228 106.51) (width 0.25) (layer F.Cu) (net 12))
 (segment (start 136.228 106.51) (end 134.62 104.902) (width 0.25) (layer F.Cu) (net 12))
 (segment (start 134.62 104.902) (end 134.62 104.14) (width 0.25) (layer F.Cu) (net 12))
 (segment (start 139.59 107.78) (end 135.72 107.78) (width 0.25) (layer F.Cu) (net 13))
 (segment (start 135.72 107.78) (end 134.62 106.68) (width 0.25) (layer F.Cu) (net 13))
 (segment (start 134.62 109.22) (end 139.42 109.22) (width 0.25) (layer F.Cu) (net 14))
 (segment (start 139.42 109.22) (end 139.59 109.05) (width 0.25) (layer F.Cu) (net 14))
 (segment (start 139.59 110.32) (end 136.06 110.32) (width 0.25) (layer F.Cu) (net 15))
 (segment (start 136.06 110.32) (end 134.62 111.76) (width 0.25) (layer F.Cu) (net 15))
 (segment (start 138.346 110.32) (end 139.59 110.32) (width 0.25) (layer F.Cu) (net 15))
 (segment (start 139.59 111.59) (end 137.33 111.59) (width 0.25) (layer F.Cu) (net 16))
 (segment (start 137.33 111.59) (end 134.62 114.3) (width 0.25) (layer F.Cu) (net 16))
 (segment (start 139.59 112.86) (end 138.6 112.86) (width 0.25) (layer F.Cu) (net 17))
 (segment (start 138.6 112.86) (end 134.62 116.84) (width 0.25) (layer F.Cu) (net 17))
 (segment (start 134.62 119.38) (end 142.748 119.38) (width 0.25) (layer F.Cu) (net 18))
 (segment (start 144.145 117.983) (end 144.145 114.35) (width 0.25) (layer F.Cu) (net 18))
 (segment (start 142.748 119.38) (end 144.145 117.983) (width 0.25) (layer F.Cu) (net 18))
 (segment (start 134.62 121.92) (end 144.145 121.92) (width 0.25) (layer F.Cu) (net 19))
 (segment (start 145.415 120.65) (end 145.415 114.35) (width 0.25) (layer F.Cu) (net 19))
 (segment (start 144.145 121.92) (end 145.415 120.65) (width 0.25) (layer F.Cu) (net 19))
 (segment (start 134.62 124.46) (end 144.653 124.46) (width 0.25) (layer F.Cu) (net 20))
 (segment (start 146.685 122.428) (end 146.685 114.35) (width 0.25) (layer F.Cu) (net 20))
 (segment (start 144.653 124.46) (end 146.685 122.428) (width 0.25) (layer F.Cu) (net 20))
 (segment (start 134.62 127) (end 145.669 127) (width 0.25) (layer F.Cu) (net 21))
 (segment (start 147.955 124.714) (end 147.955 114.35) (width 0.25) (layer F.Cu) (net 21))
 (segment (start 145.669 127) (end 147.955 124.714) (width 0.25) (layer F.Cu) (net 21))
 (segment (start 162.56 86.36) (end 159.766 89.154) (width 0.25) (layer F.Cu) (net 22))
 (segment (start 159.174 97.62) (end 157.59 97.62) (width 0.25) (layer F.Cu) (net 22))
 (segment (start 159.766 97.028) (end 159.174 97.62) (width 0.25) (layer F.Cu) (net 22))
 (segment (start 159.766 89.154) (end 159.766 97.028) (width 0.25) (layer F.Cu) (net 22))
 (segment (start 157.59 98.89) (end 159.301 98.89) (width 0.25) (layer F.Cu) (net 23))
 (segment (start 160.274 91.186) (end 162.56 88.9) (width 0.25) (layer F.Cu) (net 23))
 (segment (start 160.274 97.282) (end 160.274 91.186) (width 0.25) (layer F.Cu) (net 23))
 (segment (start 159.766 97.79) (end 160.274 97.282) (width 0.25) (layer F.Cu) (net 23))
 (segment (start 159.766 98.425) (end 159.766 97.79) (width 0.25) (layer F.Cu) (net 23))
 (segment (start 159.301 98.89) (end 159.766 98.425) (width 0.25) (layer F.Cu) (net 23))
 (segment (start 157.59 102.7) (end 159.682 102.7) (width 0.25) (layer F.Cu) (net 24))
 (segment (start 161.29 98.552) (end 162.56 97.282) (width 0.25) (layer F.Cu) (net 24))
 (segment (start 161.29 100.33) (end 161.29 98.552) (width 0.25) (layer F.Cu) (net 24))
 (segment (start 160.274 101.346) (end 161.29 100.33) (width 0.25) (layer F.Cu) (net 24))
 (segment (start 160.274 102.108) (end 160.274 101.346) (width 0.25) (layer F.Cu) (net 24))
 (segment (start 159.682 102.7) (end 160.274 102.108) (width 0.25) (layer F.Cu) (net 24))
 (segment (start 162.56 97.282) (end 162.56 96.52) (width 0.25) (layer F.Cu) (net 24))
 (segment (start 157.59 105.24) (end 160.501998 105.24) (width 0.25) (layer F.Cu) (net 25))
 (segment (start 160.782 101.6) (end 162.56 99.822) (width 0.25) (layer F.Cu) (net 25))
 (segment (start 160.782 104.959998) (end 160.782 101.6) (width 0.25) (layer F.Cu) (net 25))
 (segment (start 160.501998 105.24) (end 160.782 104.959998) (width 0.25) (layer F.Cu) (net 25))
 (segment (start 162.56 99.822) (end 162.56 99.06) (width 0.25) (layer F.Cu) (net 25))
 (segment (start 157.59 106.51) (end 160.19 106.51) (width 0.25) (layer F.Cu) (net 26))
 (segment (start 161.29 103.632) (end 162.56 102.362) (width 0.25) (layer F.Cu) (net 26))
 (segment (start 161.29 105.41) (end 161.29 103.632) (width 0.25) (layer F.Cu) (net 26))
 (segment (start 160.19 106.51) (end 161.29 105.41) (width 0.25) (layer F.Cu) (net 26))
 (segment (start 162.56 102.362) (end 162.56 101.6) (width 0.25) (layer F.Cu) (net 26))
 (segment (start 157.59 107.78) (end 159.682 107.78) (width 0.25) (layer F.Cu) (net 27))
 (segment (start 159.682 107.78) (end 162.56 104.902) (width 0.25) (layer F.Cu) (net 27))
 (segment (start 162.56 104.902) (end 162.56 104.14) (width 0.25) (layer F.Cu) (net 27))
 (segment (start 157.59 109.05) (end 160.19 109.05) (width 0.25) (layer F.Cu) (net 28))
 (segment (start 160.19 109.05) (end 162.56 106.68) (width 0.25) (layer F.Cu) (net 28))
 (segment (start 157.59 110.32) (end 161.46 110.32) (width 0.25) (layer F.Cu) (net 29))
 (segment (start 161.46 110.32) (end 162.56 109.22) (width 0.25) (layer F.Cu) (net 29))
 (segment (start 157.59 111.59) (end 157.76 111.76) (width 0.25) (layer F.Cu) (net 30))
 (segment (start 157.76 111.76) (end 162.56 111.76) (width 0.25) (layer F.Cu) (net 30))
 (segment (start 162.56 116.84) (end 154.008 116.84) (width 0.25) (layer B.Cu) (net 31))
 (segment (start 154.305 114.35) (end 154.305 115.189) (width 0.25) (layer F.Cu) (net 31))
 (segment (start 154.305 115.189) (end 155.956 116.84) (width 0.25) (layer F.Cu) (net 31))
 (segment (start 155.956 116.84) (end 162.56 116.84) (width 0.25) (layer F.Cu) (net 31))
 (segment (start 153.035 114.35) (end 153.035 117.983) (width 0.25) (layer F.Cu) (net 32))
 (segment (start 154.432 119.38) (end 162.56 119.38) (width 0.25) (layer F.Cu) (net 32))
 (segment (start 153.035 117.983) (end 154.432 119.38) (width 0.25) (layer F.Cu) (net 32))
 (segment (start 162.56 121.92) (end 153.035 121.92) (width 0.25) (layer F.Cu) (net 33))
 (segment (start 151.765 120.65) (end 151.765 114.35) (width 0.25) (layer F.Cu) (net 33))
 (segment (start 153.035 121.92) (end 151.765 120.65) (width 0.25) (layer F.Cu) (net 33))
 (segment (start 150.495 114.35) (end 150.495 122.428) (width 0.25) (layer F.Cu) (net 34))
 (segment (start 152.527 124.46) (end 162.56 124.46) (width 0.25) (layer F.Cu) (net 34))
 (segment (start 150.495 122.428) (end 152.527 124.46) (width 0.25) (layer F.Cu) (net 34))
 (segment (start 149.225 114.35) (end 149.225 124.714) (width 0.25) (layer F.Cu) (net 35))
 (segment (start 151.511 127) (end 162.56 127) (width 0.25) (layer F.Cu) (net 35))
 (segment (start 149.225 124.714) (end 151.511 127) (width 0.25) (layer F.Cu) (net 35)))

